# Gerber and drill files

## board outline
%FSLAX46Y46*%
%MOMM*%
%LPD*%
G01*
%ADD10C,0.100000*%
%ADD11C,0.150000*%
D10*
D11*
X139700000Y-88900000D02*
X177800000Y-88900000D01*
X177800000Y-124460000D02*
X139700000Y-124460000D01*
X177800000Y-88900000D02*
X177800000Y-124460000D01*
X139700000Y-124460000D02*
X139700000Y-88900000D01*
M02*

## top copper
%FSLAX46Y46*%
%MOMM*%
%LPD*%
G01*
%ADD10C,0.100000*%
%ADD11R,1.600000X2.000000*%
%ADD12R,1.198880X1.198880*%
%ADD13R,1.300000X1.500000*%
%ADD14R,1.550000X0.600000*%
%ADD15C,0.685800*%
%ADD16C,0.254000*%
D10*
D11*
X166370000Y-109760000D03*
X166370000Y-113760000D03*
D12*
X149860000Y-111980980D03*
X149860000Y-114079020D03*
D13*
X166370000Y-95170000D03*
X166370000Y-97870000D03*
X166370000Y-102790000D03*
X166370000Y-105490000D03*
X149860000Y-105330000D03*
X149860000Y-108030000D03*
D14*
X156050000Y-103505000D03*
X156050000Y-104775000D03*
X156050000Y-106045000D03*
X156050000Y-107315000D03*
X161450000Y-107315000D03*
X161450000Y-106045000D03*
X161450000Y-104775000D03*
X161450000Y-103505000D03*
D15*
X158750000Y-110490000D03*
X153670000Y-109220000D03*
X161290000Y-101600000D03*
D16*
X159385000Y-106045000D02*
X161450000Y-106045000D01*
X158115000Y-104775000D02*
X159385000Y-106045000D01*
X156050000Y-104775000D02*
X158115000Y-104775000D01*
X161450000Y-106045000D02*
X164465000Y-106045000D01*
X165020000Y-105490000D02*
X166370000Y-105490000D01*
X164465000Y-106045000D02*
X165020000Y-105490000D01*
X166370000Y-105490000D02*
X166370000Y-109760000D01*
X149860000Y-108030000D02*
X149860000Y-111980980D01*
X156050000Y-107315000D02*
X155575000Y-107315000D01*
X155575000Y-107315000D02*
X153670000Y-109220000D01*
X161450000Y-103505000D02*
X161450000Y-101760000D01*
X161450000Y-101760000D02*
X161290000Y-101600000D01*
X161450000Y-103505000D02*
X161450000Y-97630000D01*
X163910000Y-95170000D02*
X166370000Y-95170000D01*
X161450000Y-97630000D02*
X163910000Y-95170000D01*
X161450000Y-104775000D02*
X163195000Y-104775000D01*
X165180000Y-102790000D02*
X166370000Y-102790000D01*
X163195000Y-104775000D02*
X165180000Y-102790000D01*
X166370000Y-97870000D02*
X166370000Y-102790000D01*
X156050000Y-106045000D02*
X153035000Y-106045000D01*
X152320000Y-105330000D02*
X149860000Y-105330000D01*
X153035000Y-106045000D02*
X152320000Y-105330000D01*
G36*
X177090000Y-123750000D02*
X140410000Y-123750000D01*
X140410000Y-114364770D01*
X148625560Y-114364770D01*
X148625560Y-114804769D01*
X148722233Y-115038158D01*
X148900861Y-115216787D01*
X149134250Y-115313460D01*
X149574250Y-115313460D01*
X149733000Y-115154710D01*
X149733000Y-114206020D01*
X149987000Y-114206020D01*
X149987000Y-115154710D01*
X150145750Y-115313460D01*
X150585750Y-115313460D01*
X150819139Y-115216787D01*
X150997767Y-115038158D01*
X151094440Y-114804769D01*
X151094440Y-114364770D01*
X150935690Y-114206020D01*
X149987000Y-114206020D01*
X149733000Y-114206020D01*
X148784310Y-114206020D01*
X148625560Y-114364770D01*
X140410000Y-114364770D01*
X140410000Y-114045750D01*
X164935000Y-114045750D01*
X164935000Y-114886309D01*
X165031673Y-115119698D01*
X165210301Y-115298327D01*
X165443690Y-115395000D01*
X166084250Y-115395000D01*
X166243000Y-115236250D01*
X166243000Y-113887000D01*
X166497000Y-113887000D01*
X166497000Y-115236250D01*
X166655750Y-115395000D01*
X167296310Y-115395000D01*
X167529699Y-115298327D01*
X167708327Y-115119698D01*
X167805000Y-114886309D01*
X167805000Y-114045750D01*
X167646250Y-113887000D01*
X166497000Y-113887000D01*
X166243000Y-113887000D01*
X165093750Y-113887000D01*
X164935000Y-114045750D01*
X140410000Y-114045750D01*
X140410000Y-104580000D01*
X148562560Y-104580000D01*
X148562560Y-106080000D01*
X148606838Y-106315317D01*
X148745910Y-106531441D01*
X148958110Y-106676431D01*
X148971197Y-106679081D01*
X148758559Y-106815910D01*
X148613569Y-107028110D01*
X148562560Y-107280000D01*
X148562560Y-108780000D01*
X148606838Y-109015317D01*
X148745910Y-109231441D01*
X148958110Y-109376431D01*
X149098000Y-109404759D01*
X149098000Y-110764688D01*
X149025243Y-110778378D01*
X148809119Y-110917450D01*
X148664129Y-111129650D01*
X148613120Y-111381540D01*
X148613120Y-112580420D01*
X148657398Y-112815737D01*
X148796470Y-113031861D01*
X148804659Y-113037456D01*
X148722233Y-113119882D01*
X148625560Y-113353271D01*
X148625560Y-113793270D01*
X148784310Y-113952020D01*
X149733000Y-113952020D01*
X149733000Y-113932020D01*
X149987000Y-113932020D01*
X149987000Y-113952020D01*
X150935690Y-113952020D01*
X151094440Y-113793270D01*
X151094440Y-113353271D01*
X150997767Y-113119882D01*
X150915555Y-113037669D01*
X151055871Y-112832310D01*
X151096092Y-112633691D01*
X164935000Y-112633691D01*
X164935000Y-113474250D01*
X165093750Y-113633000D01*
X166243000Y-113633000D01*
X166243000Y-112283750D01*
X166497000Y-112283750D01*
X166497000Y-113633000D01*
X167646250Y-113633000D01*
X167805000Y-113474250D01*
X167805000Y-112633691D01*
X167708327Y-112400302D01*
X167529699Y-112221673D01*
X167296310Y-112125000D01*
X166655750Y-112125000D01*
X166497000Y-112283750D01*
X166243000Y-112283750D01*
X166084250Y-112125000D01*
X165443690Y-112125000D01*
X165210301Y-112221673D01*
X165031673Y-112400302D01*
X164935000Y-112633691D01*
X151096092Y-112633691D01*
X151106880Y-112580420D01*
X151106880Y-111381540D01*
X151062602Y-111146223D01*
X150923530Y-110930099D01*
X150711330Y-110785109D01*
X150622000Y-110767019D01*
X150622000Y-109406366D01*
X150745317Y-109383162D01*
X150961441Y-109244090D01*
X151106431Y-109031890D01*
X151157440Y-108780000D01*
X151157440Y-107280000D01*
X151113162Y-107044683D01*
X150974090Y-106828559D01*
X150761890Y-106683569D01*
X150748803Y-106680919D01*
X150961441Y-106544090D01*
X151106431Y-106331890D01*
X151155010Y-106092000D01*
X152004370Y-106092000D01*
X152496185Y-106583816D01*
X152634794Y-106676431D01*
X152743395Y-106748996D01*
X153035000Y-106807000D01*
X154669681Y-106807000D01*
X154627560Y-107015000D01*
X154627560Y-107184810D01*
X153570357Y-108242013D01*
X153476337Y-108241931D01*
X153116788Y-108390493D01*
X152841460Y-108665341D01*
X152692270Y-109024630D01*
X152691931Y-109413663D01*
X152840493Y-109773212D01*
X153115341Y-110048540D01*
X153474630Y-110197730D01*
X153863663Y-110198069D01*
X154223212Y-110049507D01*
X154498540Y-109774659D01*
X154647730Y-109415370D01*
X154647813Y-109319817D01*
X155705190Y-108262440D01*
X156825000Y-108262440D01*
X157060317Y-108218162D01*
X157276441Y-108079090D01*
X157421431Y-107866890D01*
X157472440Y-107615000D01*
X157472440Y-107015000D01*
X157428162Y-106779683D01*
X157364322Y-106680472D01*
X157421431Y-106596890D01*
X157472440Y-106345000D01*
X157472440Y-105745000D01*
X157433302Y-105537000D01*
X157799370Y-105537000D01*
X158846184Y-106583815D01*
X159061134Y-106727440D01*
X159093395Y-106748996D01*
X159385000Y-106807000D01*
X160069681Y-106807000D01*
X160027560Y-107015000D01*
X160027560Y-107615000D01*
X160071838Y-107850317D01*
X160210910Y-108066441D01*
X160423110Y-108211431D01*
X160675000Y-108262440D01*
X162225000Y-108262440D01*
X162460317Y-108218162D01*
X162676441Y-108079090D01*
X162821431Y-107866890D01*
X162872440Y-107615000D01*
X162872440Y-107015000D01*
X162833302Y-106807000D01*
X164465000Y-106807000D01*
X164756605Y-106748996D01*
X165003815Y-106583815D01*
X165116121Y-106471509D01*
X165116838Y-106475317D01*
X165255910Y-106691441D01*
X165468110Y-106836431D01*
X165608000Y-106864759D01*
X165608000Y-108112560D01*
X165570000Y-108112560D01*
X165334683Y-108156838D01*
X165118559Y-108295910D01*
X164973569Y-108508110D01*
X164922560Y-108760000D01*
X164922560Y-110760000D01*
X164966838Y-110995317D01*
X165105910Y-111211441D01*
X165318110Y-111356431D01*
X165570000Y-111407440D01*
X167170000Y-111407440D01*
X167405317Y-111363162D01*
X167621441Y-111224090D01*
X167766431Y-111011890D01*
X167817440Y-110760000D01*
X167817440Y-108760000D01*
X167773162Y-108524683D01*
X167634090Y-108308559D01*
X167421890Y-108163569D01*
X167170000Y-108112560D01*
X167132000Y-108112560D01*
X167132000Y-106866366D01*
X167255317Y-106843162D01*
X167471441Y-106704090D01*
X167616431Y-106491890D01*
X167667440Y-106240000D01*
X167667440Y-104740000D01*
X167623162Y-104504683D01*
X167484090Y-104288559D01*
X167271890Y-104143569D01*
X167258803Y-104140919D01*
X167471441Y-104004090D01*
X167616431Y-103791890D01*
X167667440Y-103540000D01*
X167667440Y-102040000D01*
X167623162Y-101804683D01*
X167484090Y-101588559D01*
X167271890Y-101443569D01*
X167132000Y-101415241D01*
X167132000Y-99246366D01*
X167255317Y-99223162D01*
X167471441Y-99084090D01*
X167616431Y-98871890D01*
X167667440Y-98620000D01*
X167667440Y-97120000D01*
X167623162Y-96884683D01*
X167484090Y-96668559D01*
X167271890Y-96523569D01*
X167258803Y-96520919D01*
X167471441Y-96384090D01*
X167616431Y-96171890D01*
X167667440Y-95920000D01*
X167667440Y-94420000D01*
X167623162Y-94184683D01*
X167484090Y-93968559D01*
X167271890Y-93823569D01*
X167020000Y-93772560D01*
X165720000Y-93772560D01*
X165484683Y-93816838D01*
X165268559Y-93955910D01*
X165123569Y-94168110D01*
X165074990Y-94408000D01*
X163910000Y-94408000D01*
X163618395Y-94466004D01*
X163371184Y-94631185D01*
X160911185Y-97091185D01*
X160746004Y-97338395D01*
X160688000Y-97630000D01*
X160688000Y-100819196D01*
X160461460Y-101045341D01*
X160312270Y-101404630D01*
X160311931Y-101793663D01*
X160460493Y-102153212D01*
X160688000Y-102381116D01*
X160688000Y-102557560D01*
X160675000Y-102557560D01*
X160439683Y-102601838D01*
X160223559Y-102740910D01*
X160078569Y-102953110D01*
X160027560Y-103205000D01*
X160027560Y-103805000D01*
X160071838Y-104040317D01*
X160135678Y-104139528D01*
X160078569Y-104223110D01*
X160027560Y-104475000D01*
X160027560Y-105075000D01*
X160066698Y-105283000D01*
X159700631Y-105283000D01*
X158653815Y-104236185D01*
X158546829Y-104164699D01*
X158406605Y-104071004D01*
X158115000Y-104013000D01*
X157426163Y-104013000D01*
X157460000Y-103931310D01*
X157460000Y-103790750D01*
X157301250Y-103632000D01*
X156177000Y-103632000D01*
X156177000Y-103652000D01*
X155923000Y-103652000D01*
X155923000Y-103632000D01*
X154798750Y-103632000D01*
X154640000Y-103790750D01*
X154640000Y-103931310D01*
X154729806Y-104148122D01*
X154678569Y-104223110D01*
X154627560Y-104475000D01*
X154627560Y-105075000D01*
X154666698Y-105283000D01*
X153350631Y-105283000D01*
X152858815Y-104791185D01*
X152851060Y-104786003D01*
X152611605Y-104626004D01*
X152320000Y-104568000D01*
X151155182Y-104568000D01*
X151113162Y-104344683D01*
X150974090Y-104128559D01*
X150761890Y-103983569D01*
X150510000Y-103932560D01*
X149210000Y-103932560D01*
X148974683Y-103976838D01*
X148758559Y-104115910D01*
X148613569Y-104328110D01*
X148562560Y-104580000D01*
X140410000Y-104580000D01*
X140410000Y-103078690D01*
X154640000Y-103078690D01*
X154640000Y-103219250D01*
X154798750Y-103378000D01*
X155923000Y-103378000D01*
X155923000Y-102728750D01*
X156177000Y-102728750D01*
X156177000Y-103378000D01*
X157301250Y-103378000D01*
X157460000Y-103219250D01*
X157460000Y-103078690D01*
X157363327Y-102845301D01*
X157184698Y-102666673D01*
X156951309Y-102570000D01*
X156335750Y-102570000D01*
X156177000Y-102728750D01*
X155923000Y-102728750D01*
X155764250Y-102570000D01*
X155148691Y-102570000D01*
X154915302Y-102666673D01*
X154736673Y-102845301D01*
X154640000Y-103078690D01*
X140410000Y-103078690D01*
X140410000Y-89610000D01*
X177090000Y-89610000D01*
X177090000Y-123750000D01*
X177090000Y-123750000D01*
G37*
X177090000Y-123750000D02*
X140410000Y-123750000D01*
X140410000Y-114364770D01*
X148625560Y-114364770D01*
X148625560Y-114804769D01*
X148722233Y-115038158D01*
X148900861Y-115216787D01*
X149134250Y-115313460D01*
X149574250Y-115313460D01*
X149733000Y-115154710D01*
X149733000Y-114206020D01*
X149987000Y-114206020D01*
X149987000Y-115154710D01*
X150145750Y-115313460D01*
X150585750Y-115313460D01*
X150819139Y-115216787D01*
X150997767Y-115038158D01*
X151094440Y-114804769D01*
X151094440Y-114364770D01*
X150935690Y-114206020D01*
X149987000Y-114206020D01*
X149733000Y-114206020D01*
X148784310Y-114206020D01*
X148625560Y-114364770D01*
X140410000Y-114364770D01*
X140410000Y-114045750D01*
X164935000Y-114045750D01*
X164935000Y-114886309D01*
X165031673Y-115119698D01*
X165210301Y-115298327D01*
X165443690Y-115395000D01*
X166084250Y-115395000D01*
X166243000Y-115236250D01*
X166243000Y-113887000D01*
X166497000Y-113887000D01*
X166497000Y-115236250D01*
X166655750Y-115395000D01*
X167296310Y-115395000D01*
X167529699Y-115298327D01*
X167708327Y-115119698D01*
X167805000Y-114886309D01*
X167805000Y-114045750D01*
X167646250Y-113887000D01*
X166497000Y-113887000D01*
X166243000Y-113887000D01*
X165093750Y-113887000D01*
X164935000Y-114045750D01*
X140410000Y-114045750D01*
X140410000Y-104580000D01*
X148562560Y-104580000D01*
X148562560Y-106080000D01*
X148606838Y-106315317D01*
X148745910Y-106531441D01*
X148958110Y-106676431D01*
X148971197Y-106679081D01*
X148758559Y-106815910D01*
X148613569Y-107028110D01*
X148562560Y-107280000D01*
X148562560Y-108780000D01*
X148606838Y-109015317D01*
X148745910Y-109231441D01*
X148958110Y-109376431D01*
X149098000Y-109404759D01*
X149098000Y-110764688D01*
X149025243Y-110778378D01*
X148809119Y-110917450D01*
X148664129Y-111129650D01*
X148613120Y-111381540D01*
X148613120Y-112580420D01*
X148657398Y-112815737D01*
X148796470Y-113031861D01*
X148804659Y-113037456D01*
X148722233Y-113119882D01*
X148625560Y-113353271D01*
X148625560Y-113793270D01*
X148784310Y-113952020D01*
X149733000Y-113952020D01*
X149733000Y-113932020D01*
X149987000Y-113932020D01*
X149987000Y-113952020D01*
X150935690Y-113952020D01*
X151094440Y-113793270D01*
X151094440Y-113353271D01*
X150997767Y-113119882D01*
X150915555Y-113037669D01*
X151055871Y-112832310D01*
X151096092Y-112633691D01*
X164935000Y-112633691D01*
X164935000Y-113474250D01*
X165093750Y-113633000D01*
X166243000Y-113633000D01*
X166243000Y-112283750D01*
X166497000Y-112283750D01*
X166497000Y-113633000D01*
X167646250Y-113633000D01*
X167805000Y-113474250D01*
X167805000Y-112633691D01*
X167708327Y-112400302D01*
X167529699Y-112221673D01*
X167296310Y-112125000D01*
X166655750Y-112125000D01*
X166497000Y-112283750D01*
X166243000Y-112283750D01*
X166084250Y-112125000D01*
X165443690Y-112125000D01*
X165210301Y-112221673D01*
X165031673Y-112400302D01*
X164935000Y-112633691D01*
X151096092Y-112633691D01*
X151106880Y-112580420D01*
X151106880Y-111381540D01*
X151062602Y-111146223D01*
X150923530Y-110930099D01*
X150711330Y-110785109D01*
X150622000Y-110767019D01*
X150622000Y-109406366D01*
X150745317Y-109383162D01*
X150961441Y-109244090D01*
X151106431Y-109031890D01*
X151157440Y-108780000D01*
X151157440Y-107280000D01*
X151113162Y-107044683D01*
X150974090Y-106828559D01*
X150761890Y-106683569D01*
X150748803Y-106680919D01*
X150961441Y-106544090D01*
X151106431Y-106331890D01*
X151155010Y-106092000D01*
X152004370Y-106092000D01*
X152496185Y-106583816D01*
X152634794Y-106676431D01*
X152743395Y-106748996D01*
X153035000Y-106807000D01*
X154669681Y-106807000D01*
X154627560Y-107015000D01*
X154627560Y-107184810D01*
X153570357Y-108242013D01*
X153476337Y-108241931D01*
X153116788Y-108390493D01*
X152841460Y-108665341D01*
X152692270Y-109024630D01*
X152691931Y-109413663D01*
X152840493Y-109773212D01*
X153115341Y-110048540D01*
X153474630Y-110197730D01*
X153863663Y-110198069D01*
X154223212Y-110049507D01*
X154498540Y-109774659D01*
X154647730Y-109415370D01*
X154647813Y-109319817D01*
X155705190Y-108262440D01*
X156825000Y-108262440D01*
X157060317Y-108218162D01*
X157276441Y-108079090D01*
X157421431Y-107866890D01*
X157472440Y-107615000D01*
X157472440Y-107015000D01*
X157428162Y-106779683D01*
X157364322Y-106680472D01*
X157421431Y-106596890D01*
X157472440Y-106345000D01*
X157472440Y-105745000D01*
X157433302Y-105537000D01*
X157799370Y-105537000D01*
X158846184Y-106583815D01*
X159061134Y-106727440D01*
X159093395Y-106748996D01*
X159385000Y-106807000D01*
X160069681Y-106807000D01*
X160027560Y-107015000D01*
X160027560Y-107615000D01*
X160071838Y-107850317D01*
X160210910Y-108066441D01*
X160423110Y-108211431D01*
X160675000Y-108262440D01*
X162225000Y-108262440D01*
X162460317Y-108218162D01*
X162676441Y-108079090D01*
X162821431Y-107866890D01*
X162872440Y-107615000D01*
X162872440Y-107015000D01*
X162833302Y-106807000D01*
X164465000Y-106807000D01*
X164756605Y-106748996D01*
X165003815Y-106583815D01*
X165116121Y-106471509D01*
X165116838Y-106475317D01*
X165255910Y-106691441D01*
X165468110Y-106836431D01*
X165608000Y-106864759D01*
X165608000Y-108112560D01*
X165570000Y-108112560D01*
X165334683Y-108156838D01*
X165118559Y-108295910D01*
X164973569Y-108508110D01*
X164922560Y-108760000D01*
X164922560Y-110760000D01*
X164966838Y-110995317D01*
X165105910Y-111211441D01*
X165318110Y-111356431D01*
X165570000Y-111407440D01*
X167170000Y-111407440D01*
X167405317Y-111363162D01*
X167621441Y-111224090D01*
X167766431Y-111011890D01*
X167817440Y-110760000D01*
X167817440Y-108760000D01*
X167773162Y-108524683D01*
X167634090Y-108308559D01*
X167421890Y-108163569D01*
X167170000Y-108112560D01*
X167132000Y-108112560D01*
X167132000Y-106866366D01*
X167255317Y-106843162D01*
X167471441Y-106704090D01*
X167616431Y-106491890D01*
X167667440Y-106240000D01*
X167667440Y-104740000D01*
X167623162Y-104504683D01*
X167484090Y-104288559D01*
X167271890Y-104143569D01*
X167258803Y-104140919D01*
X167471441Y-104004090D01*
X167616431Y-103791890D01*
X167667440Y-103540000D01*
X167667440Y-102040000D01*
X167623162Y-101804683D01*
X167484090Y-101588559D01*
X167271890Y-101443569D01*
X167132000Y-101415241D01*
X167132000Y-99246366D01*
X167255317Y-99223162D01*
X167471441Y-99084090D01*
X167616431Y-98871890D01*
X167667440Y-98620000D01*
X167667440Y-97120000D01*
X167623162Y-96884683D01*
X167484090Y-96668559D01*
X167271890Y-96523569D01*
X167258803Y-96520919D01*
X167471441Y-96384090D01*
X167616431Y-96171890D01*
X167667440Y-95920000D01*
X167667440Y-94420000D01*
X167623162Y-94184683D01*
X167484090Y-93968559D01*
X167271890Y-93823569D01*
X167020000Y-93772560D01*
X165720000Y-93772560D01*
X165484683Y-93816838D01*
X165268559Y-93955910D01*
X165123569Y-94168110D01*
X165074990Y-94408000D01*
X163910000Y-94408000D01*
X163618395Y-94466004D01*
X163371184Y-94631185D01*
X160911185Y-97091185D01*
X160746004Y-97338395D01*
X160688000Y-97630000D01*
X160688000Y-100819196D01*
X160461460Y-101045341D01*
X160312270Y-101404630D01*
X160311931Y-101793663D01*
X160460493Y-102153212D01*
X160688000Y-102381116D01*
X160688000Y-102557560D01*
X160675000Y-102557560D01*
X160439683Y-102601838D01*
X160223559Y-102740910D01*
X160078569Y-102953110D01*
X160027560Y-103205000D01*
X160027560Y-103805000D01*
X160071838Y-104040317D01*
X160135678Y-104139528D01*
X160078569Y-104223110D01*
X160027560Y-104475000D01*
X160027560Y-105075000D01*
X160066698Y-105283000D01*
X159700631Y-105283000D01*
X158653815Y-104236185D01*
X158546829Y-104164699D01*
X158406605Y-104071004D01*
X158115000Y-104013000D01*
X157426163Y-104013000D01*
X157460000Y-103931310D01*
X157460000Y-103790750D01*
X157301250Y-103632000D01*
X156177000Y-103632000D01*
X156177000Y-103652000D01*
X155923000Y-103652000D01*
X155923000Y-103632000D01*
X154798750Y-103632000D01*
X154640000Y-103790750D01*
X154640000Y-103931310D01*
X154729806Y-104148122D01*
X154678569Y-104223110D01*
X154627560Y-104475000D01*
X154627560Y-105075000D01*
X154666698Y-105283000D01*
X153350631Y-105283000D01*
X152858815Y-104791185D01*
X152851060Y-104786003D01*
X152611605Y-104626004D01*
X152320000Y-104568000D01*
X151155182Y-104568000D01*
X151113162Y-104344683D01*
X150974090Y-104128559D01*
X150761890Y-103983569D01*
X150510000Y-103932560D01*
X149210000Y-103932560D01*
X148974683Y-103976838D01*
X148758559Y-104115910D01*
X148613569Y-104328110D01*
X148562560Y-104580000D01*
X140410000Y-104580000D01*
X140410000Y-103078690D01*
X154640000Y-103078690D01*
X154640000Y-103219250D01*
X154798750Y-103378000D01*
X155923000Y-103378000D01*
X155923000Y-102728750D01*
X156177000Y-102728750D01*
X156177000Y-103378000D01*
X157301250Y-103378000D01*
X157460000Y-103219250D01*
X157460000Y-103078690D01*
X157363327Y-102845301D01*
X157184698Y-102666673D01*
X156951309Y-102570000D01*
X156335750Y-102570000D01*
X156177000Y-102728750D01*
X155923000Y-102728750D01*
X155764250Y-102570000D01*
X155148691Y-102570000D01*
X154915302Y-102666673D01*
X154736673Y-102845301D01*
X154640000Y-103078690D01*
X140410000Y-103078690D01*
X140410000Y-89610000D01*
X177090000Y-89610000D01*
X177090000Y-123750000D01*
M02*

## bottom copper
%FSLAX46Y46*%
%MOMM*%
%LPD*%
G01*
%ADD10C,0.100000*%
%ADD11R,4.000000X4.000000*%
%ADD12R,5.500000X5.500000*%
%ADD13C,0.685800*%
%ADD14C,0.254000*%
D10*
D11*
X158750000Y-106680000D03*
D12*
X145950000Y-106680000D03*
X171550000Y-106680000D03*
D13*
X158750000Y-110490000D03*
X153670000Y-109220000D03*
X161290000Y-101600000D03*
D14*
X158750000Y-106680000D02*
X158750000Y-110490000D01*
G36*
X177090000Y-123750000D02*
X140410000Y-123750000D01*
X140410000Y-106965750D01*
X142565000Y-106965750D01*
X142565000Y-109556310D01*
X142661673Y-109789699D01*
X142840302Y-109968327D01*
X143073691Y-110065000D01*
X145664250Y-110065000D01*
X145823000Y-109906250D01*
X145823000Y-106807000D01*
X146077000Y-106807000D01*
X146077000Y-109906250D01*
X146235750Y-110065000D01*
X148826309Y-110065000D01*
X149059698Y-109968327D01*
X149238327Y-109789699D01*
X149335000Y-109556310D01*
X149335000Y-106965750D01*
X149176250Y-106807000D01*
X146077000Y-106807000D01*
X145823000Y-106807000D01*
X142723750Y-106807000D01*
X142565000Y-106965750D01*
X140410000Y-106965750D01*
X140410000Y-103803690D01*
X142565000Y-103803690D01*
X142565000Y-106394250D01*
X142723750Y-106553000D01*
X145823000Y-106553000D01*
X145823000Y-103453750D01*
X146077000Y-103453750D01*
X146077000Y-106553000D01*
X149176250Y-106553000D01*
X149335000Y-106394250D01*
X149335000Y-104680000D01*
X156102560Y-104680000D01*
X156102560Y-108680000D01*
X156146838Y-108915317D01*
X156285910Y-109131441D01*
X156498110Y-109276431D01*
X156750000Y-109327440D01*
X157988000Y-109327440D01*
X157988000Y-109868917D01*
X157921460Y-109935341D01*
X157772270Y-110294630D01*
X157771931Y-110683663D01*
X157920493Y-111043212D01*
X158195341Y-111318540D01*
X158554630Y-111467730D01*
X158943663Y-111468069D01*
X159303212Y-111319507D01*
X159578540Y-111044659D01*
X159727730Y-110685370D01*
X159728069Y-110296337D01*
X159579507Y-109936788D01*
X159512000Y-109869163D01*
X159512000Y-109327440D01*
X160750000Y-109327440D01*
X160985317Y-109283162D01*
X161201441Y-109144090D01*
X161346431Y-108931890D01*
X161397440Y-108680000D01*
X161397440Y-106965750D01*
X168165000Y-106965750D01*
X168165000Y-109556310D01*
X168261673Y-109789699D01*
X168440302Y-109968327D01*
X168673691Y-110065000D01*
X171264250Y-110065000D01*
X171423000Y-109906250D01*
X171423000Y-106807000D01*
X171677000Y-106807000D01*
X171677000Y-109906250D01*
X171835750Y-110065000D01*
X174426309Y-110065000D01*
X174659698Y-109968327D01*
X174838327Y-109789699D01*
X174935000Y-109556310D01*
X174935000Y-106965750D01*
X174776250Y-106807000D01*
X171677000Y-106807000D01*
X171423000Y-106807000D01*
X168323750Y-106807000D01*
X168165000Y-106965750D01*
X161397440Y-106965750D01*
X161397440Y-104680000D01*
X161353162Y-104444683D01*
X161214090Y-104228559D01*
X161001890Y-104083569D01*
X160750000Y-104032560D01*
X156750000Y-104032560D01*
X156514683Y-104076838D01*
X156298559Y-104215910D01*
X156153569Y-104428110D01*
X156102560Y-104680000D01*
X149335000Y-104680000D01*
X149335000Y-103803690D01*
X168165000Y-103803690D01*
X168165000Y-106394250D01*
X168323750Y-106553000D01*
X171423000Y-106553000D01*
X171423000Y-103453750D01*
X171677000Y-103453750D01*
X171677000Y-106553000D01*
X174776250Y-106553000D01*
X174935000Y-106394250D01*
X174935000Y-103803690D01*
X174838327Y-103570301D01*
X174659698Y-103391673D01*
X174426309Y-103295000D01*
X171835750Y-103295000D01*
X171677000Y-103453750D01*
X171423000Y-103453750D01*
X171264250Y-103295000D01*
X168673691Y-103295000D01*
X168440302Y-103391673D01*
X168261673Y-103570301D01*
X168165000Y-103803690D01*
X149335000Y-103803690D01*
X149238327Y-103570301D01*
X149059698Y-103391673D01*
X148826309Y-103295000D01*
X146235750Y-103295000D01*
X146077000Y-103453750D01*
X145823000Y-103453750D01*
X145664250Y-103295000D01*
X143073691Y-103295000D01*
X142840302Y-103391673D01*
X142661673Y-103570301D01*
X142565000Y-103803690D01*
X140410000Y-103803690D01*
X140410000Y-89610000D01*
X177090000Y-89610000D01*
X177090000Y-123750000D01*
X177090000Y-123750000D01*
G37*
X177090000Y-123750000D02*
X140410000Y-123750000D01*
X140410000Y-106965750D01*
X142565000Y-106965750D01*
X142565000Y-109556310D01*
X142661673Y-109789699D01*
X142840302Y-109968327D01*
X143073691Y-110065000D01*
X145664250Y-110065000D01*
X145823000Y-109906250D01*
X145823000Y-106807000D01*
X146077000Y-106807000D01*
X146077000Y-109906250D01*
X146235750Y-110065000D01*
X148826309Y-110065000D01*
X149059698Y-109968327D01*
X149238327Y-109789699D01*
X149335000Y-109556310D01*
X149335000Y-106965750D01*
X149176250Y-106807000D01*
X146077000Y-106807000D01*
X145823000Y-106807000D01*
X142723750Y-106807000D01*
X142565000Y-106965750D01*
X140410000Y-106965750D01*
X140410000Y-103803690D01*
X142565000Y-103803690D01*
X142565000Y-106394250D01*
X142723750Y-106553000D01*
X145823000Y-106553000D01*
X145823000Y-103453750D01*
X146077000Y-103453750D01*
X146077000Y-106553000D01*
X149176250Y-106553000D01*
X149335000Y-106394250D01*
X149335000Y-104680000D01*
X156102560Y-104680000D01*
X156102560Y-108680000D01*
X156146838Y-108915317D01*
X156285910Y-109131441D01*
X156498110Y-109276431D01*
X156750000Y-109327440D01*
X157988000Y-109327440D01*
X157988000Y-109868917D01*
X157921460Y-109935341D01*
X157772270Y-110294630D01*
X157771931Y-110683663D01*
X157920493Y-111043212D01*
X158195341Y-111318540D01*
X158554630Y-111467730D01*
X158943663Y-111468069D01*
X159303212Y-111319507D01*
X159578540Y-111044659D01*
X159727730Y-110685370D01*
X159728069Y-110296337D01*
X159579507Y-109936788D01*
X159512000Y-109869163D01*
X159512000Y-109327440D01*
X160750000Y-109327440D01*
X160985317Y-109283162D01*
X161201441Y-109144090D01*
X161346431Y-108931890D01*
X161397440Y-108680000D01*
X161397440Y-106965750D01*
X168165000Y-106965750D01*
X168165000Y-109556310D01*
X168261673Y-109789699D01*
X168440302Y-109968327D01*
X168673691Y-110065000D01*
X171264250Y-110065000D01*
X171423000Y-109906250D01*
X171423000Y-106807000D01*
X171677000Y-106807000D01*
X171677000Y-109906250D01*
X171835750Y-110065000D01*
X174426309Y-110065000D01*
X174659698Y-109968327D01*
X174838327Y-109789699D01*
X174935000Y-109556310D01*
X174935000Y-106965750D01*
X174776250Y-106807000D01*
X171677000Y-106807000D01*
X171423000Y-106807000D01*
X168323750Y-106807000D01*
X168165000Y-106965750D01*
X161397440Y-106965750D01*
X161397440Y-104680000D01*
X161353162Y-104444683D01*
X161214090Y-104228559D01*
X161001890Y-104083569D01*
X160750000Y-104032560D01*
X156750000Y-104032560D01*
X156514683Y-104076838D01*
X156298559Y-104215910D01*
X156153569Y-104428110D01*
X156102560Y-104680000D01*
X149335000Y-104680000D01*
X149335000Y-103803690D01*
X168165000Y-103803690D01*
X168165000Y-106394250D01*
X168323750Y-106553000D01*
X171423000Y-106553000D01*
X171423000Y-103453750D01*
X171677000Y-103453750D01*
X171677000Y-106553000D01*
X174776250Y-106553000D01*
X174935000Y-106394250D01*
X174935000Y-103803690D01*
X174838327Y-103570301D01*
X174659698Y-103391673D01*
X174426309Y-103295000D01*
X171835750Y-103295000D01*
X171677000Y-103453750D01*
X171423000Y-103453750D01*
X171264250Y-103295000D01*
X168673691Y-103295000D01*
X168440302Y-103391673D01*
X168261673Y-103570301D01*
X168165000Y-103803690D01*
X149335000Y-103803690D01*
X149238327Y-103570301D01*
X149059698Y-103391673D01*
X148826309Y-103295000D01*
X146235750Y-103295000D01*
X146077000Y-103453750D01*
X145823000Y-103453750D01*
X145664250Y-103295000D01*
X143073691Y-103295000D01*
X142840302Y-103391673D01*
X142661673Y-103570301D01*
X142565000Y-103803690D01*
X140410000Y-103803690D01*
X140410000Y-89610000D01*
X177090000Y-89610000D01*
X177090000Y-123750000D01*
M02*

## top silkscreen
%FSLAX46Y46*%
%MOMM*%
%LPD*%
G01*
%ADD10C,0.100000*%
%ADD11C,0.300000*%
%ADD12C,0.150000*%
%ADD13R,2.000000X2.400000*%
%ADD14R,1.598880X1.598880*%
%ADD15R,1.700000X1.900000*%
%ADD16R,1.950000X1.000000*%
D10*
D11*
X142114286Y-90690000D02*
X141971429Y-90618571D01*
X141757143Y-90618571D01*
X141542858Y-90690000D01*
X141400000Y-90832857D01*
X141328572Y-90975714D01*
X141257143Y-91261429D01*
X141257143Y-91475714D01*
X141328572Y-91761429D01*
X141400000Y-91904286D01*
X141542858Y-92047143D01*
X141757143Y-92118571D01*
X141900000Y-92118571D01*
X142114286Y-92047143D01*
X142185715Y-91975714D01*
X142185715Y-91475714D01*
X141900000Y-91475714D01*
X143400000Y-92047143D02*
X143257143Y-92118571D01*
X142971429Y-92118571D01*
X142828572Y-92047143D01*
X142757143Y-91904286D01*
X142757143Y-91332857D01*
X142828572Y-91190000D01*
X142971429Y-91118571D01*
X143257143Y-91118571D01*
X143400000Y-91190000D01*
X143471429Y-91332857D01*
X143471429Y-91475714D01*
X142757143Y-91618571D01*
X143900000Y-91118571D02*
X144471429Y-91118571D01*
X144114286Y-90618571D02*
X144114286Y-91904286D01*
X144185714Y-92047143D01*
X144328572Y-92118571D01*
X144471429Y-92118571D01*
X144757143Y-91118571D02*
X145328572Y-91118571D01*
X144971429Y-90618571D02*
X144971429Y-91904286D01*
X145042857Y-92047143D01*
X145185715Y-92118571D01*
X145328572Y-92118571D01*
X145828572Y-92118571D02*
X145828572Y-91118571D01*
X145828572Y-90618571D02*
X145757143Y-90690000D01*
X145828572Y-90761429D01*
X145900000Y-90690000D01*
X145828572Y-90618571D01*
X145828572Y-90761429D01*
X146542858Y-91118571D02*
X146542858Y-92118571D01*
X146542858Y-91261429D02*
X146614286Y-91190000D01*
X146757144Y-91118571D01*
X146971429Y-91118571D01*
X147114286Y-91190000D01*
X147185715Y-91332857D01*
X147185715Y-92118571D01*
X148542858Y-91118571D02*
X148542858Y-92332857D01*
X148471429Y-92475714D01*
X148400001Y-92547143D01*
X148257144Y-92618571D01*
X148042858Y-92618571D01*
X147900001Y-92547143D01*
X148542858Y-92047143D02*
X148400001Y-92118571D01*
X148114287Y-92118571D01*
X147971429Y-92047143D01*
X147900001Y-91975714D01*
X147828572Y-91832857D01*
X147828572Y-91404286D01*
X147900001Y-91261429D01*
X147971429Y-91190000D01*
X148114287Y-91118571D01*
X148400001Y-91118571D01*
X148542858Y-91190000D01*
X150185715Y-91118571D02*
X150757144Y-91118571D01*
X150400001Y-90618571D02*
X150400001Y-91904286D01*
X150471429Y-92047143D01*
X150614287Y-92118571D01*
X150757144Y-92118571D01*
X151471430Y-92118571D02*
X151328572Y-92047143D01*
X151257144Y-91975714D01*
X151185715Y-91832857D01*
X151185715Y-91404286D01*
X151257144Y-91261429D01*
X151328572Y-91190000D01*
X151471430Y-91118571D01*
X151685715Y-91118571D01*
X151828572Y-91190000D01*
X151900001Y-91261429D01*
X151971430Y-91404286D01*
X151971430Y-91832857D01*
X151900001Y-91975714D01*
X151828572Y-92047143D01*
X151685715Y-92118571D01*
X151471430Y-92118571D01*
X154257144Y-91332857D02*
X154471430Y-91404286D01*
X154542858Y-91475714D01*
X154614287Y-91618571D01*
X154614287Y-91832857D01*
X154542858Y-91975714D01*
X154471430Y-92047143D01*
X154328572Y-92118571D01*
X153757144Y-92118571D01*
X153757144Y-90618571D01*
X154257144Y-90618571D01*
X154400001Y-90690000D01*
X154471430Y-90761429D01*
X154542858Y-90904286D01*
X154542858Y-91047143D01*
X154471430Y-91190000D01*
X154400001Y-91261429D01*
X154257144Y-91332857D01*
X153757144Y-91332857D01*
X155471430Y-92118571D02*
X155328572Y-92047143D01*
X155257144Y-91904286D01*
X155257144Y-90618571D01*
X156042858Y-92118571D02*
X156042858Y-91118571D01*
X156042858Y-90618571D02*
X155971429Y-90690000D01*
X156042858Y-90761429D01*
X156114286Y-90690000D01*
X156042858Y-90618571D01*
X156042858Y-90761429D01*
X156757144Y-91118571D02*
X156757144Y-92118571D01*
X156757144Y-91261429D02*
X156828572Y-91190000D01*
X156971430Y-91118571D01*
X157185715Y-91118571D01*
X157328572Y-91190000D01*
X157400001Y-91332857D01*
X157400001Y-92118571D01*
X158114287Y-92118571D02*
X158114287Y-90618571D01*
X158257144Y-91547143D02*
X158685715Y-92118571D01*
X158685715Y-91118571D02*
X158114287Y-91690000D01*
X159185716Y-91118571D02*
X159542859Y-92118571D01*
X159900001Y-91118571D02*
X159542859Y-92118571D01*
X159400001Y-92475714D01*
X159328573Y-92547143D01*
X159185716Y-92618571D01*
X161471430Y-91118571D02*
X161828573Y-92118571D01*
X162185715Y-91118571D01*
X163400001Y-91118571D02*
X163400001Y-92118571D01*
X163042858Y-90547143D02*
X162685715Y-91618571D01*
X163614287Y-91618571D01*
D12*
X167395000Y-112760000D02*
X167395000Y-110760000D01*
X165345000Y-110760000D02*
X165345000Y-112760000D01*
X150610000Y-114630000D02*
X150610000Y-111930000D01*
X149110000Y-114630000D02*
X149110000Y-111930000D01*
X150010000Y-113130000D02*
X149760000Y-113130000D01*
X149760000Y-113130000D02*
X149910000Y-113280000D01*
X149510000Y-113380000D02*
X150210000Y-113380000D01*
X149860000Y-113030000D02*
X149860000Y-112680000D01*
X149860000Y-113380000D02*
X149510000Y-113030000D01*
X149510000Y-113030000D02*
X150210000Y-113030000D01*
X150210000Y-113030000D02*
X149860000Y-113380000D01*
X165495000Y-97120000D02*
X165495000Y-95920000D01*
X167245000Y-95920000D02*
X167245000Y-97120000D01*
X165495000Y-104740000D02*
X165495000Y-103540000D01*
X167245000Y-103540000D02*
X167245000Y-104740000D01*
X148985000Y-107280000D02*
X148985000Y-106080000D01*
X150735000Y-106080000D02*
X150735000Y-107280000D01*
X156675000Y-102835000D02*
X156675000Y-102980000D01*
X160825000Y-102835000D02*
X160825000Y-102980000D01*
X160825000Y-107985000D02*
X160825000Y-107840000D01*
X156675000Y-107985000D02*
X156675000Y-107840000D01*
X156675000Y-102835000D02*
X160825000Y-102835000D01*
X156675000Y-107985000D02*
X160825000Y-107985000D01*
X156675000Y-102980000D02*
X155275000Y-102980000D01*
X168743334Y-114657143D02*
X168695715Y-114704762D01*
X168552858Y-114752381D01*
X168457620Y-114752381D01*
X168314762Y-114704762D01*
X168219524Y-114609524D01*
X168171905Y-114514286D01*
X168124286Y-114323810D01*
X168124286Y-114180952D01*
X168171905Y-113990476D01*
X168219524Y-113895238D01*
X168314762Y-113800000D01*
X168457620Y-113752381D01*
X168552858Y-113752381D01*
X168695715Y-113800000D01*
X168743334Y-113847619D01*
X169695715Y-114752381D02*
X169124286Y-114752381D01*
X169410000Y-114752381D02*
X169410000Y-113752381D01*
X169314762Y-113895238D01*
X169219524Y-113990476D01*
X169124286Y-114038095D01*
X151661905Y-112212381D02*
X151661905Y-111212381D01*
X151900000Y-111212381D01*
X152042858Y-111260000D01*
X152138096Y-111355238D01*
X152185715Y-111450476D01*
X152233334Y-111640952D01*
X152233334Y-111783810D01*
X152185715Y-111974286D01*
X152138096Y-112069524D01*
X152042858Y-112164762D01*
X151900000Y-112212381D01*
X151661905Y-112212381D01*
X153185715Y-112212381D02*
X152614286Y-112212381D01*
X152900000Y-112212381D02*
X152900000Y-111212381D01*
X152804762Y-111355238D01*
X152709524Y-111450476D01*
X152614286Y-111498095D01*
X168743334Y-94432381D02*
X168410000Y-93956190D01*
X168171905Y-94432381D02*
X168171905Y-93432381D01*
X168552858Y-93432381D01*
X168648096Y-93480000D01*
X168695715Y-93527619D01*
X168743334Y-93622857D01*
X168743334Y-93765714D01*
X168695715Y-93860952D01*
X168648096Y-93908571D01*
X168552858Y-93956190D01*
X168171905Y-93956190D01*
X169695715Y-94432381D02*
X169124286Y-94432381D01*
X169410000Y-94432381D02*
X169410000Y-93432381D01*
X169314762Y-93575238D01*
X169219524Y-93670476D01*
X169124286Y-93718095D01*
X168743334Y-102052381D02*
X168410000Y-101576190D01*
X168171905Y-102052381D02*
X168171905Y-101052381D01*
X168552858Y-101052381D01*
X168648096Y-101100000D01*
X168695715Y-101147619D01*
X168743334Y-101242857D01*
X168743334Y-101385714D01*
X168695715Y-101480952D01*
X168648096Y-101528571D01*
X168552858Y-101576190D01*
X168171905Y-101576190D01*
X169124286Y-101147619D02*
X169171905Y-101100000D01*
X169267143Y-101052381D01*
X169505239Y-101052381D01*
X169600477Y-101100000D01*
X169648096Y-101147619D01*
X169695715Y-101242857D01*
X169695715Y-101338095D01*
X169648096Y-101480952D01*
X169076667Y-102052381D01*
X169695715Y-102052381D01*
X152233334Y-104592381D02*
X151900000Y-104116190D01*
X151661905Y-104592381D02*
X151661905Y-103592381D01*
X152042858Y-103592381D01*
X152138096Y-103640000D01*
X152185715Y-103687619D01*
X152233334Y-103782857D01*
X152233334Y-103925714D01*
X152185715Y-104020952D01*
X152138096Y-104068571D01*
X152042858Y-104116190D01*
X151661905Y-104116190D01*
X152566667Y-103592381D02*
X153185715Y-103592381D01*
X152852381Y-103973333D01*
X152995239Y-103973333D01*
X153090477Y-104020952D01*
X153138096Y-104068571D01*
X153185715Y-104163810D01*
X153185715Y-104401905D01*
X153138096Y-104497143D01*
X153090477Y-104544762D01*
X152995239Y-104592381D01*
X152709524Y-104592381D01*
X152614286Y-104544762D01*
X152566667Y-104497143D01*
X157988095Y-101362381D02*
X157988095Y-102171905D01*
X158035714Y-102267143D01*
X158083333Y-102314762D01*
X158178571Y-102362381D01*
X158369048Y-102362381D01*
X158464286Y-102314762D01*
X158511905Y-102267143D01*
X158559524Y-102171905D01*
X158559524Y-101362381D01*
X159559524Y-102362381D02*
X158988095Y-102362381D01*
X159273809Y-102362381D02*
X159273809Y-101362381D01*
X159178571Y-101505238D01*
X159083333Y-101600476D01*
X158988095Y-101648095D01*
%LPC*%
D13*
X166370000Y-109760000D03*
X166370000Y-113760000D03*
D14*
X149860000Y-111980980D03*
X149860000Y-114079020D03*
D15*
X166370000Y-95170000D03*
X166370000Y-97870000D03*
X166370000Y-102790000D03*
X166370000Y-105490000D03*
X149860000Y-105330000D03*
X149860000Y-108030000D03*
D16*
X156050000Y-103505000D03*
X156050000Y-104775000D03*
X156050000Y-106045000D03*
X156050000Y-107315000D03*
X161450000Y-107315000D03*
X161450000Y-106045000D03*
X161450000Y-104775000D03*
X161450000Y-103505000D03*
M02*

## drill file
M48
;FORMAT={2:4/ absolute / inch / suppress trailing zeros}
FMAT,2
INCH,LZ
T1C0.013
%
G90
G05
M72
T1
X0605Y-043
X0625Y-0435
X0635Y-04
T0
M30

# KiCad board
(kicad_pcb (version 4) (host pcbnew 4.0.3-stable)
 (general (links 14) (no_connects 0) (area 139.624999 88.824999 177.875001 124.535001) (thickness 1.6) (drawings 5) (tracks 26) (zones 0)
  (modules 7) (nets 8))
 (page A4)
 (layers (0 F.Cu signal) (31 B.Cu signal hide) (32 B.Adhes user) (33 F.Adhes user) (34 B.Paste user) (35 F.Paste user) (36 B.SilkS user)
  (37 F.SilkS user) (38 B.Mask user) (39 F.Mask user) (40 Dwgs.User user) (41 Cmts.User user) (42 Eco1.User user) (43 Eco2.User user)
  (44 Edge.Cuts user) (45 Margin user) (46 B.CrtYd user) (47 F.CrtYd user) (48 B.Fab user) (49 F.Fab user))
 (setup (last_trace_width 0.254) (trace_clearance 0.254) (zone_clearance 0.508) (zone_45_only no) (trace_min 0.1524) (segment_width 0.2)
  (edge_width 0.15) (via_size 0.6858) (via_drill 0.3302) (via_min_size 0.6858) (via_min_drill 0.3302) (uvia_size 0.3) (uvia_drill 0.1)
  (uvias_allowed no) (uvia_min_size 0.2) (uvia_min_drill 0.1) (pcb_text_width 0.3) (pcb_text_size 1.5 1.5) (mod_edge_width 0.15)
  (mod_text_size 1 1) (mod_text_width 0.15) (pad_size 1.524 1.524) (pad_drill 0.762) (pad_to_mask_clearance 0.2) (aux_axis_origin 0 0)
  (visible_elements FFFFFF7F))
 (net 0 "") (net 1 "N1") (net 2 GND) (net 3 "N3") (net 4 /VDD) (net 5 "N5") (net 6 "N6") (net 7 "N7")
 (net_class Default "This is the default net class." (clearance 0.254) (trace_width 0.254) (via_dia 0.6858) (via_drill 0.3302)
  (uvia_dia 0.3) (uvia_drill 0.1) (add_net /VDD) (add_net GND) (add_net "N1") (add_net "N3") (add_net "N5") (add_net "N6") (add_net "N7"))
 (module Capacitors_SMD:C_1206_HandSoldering (layer F.Cu) (at 166.37 111.76 270)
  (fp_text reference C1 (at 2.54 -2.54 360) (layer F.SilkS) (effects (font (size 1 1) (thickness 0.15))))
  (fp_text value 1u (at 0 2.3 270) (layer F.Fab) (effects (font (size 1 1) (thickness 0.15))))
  (fp_line (start 1 -1.025) (end -1 -1.025) (layer F.SilkS) (width 0.15))
  (fp_line (start -1 1.025) (end 1 1.025) (layer F.SilkS) (width 0.15))
  (pad 1 smd rect (at -2 0 270) (size 2 1.6) (layers F.Cu F.Paste F.Mask) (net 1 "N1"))
  (pad 2 smd rect (at 2 0 270) (size 2 1.6) (layers F.Cu F.Paste F.Mask) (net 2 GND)))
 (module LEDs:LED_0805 (layer F.Cu) (at 149.86 113.03 90)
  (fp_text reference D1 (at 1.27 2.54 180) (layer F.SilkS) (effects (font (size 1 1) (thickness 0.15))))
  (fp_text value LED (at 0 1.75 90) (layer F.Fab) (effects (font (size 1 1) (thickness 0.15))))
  (fp_line (start -1.6 0.75) (end 1.1 0.75) (layer F.SilkS) (width 0.15))
  (fp_line (start -1.6 -0.75) (end 1.1 -0.75) (layer F.SilkS) (width 0.15))
  (fp_line (start -0.1 0.15) (end -0.1 -0.1) (layer F.SilkS) (width 0.15))
  (fp_line (start -0.1 -0.1) (end -0.25 0.05) (layer F.SilkS) (width 0.15))
  (fp_line (start -0.35 -0.35) (end -0.35 0.35) (layer F.SilkS) (width 0.15))
  (fp_line (start 0 0) (end 0.35 0) (layer F.SilkS) (width 0.15))
  (fp_line (start -0.35 0) (end 0 -0.35) (layer F.SilkS) (width 0.15))
  (fp_line (start 0 -0.35) (end 0 0.35) (layer F.SilkS) (width 0.15))
  (fp_line (start 0 0.35) (end -0.35 0) (layer F.SilkS) (width 0.15))
  (pad 2 smd rect (at 1.04902 0 270) (size 1.19888 1.19888) (layers F.Cu F.Paste F.Mask) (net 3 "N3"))
  (pad 1 smd rect (at -1.04902 0 270) (size 1.19888 1.19888) (layers F.Cu F.Paste F.Mask) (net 2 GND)))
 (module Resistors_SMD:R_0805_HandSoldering (layer F.Cu) (at 166.37 96.52 270)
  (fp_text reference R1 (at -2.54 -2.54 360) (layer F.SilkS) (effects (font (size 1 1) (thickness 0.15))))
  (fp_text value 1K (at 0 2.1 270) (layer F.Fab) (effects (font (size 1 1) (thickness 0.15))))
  (fp_line (start 0.6 0.875) (end -0.6 0.875) (layer F.SilkS) (width 0.15))
  (fp_line (start -0.6 -0.875) (end 0.6 -0.875) (layer F.SilkS) (width 0.15))
  (pad 1 smd rect (at -1.35 0 270) (size 1.5 1.3) (layers F.Cu F.Paste F.Mask) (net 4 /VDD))
  (pad 2 smd rect (at 1.35 0 270) (size 1.5 1.3) (layers F.Cu F.Paste F.Mask) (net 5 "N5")))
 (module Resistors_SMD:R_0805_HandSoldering (layer F.Cu) (at 166.37 104.14 270)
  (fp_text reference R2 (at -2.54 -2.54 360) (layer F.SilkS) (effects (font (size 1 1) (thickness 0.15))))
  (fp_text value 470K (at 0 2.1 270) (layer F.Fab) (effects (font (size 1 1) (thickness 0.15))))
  (fp_line (start 0.6 0.875) (end -0.6 0.875) (layer F.SilkS) (width 0.15))
  (fp_line (start -0.6 -0.875) (end 0.6 -0.875) (layer F.SilkS) (width 0.15))
  (pad 1 smd rect (at -1.35 0 270) (size 1.5 1.3) (layers F.Cu F.Paste F.Mask) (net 5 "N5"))
  (pad 2 smd rect (at 1.35 0 270) (size 1.5 1.3) (layers F.Cu F.Paste F.Mask) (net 1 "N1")))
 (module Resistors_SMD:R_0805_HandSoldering (layer F.Cu) (at 149.86 106.68 270)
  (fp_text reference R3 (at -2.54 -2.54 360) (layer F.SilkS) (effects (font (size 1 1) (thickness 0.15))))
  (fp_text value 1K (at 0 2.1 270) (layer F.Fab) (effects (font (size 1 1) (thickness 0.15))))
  (fp_line (start 0.6 0.875) (end -0.6 0.875) (layer F.SilkS) (width 0.15))
  (fp_line (start -0.6 -0.875) (end 0.6 -0.875) (layer F.SilkS) (width 0.15))
  (pad 1 smd rect (at -1.35 0 270) (size 1.5 1.3) (layers F.Cu F.Paste F.Mask) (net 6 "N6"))
  (pad 2 smd rect (at 1.35 0 270) (size 1.5 1.3) (layers F.Cu F.Paste F.Mask) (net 3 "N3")))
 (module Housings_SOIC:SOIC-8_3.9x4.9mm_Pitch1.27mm (layer F.Cu) (at 158.75 105.41)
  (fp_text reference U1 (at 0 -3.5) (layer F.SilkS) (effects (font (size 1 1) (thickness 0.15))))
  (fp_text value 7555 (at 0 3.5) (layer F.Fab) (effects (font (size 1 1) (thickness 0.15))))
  (fp_line (start -2.075 -2.575) (end -2.075 -2.43) (layer F.SilkS) (width 0.15))
  (fp_line (start 2.075 -2.575) (end 2.075 -2.43) (layer F.SilkS) (width 0.15))
  (fp_line (start 2.075 2.575) (end 2.075 2.43) (layer F.SilkS) (width 0.15))
  (fp_line (start -2.075 2.575) (end -2.075 2.43) (layer F.SilkS) (width 0.15))
  (fp_line (start -2.075 -2.575) (end 2.075 -2.575) (layer F.SilkS) (width 0.15))
  (fp_line (start -2.075 2.575) (end 2.075 2.575) (layer F.SilkS) (width 0.15))
  (fp_line (start -2.075 -2.43) (end -3.475 -2.43) (layer F.SilkS) (width 0.15))
  (pad 1 smd rect (at -2.7 -1.905) (size 1.55 0.6) (layers F.Cu F.Paste F.Mask) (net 2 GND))
  (pad 2 smd rect (at -2.7 -0.635) (size 1.55 0.6) (layers F.Cu F.Paste F.Mask) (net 1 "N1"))
  (pad 3 smd rect (at -2.7 0.635) (size 1.55 0.6) (layers F.Cu F.Paste F.Mask) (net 6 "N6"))
  (pad 4 smd rect (at -2.7 1.905) (size 1.55 0.6) (layers F.Cu F.Paste F.Mask) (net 4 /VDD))
  (pad 5 smd rect (at 2.7 1.905) (size 1.55 0.6) (layers F.Cu F.Paste F.Mask) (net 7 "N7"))
  (pad 6 smd rect (at 2.7 0.635) (size 1.55 0.6) (layers F.Cu F.Paste F.Mask) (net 1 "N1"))
  (pad 7 smd rect (at 2.7 -0.635) (size 1.55 0.6) (layers F.Cu F.Paste F.Mask) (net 5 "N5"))
  (pad 8 smd rect (at 2.7 -1.905) (size 1.55 0.6) (layers F.Cu F.Paste F.Mask) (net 4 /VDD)))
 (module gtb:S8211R (layer B.Cu) (at 158.75 106.68)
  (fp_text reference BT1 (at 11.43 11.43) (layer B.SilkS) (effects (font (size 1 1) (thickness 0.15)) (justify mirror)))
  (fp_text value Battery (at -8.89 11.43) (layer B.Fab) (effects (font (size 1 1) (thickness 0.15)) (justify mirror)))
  (pad 2 smd rect (at 0 0) (size 4 4) (layers B.Cu B.Paste B.Mask) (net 2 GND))
  (pad 1 smd rect (at -12.8 0) (size 5.5 5.5) (layers B.Cu B.Paste B.Mask) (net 4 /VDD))
  (pad 1 smd rect (at 12.8 0) (size 5.5 5.5) (layers B.Cu B.Paste B.Mask) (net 4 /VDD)))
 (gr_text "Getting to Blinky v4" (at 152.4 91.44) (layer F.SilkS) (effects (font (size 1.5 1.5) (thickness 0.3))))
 (gr_line (start 139.7 88.9) (end 177.8 88.9) (angle 90) (layer Edge.Cuts) (width 0.15))
 (gr_line (start 177.8 124.46) (end 139.7 124.46) (angle 90) (layer Edge.Cuts) (width 0.15))
 (gr_line (start 177.8 88.9) (end 177.8 124.46) (angle 90) (layer Edge.Cuts) (width 0.15))
 (gr_line (start 139.7 124.46) (end 139.7 88.9) (angle 90) (layer Edge.Cuts) (width 0.15))
 (segment (start 159.385 106.045) (end 161.45 106.045) (width 0.254) (layer F.Cu) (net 1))
 (segment (start 158.115 104.775) (end 159.385 106.045) (width 0.254) (layer F.Cu) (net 1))
 (segment (start 156.05 104.775) (end 158.115 104.775) (width 0.254) (layer F.Cu) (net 1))
 (segment (start 161.45 106.045) (end 164.465 106.045) (width 0.254) (layer F.Cu) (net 1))
 (segment (start 165.02 105.49) (end 166.37 105.49) (width 0.254) (layer F.Cu) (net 1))
 (segment (start 164.465 106.045) (end 165.02 105.49) (width 0.254) (layer F.Cu) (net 1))
 (segment (start 166.37 105.49) (end 166.37 109.76) (width 0.254) (layer F.Cu) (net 1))
 (segment (start 158.75 106.68) (end 158.75 110.49) (width 0.254) (layer B.Cu) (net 2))
 (via (at 158.75 110.49) (size 0.6858) (drill 0.3302) (layers F.Cu B.Cu) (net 2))
 (segment (start 149.86 108.03) (end 149.86 111.98098) (width 0.254) (layer F.Cu) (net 3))
 (segment (start 156.05 107.315) (end 155.575 107.315) (width 0.254) (layer F.Cu) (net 4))
 (segment (start 155.575 107.315) (end 153.67 109.22) (width 0.254) (layer F.Cu) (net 4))
 (via (at 153.67 109.22) (size 0.6858) (drill 0.3302) (layers F.Cu B.Cu) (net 4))
 (segment (start 161.45 103.505) (end 161.45 101.76) (width 0.254) (layer F.Cu) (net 4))
 (via (at 161.29 101.6) (size 0.6858) (drill 0.3302) (layers F.Cu B.Cu) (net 4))
 (segment (start 161.45 101.76) (end 161.29 101.6) (width 0.254) (layer F.Cu) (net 4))
 (segment (start 161.45 103.505) (end 161.45 97.63) (width 0.254) (layer F.Cu) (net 4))
 (segment (start 163.91 95.17) (end 166.37 95.17) (width 0.254) (layer F.Cu) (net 4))
 (segment (start 161.45 97.63) (end 163.91 95.17) (width 0.254) (layer F.Cu) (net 4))
 (segment (start 161.45 104.775) (end 163.195 104.775) (width 0.254) (layer F.Cu) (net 5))
 (segment (start 165.18 102.79) (end 166.37 102.79) (width 0.254) (layer F.Cu) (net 5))
 (segment (start 163.195 104.775) (end 165.18 102.79) (width 0.254) (layer F.Cu) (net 5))
 (segment (start 166.37 97.87) (end 166.37 102.79) (width 0.254) (layer F.Cu) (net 5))
 (segment (start 156.05 106.045) (end 153.035 106.045) (width 0.254) (layer F.Cu) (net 6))
 (segment (start 152.32 105.33) (end 149.86 105.33) (width 0.254) (layer F.Cu) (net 6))
 (segment (start 153.035 106.045) (end 152.32 105.33) (width 0.254) (layer F.Cu) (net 6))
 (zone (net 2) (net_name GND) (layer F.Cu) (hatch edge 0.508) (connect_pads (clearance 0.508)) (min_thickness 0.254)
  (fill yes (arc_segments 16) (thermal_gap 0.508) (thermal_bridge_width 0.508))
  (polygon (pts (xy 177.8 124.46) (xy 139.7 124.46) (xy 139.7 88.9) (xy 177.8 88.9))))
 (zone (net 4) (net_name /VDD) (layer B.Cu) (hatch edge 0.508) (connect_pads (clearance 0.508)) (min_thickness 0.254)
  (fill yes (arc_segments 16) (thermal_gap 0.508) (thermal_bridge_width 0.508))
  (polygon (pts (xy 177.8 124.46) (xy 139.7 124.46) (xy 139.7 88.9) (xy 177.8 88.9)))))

